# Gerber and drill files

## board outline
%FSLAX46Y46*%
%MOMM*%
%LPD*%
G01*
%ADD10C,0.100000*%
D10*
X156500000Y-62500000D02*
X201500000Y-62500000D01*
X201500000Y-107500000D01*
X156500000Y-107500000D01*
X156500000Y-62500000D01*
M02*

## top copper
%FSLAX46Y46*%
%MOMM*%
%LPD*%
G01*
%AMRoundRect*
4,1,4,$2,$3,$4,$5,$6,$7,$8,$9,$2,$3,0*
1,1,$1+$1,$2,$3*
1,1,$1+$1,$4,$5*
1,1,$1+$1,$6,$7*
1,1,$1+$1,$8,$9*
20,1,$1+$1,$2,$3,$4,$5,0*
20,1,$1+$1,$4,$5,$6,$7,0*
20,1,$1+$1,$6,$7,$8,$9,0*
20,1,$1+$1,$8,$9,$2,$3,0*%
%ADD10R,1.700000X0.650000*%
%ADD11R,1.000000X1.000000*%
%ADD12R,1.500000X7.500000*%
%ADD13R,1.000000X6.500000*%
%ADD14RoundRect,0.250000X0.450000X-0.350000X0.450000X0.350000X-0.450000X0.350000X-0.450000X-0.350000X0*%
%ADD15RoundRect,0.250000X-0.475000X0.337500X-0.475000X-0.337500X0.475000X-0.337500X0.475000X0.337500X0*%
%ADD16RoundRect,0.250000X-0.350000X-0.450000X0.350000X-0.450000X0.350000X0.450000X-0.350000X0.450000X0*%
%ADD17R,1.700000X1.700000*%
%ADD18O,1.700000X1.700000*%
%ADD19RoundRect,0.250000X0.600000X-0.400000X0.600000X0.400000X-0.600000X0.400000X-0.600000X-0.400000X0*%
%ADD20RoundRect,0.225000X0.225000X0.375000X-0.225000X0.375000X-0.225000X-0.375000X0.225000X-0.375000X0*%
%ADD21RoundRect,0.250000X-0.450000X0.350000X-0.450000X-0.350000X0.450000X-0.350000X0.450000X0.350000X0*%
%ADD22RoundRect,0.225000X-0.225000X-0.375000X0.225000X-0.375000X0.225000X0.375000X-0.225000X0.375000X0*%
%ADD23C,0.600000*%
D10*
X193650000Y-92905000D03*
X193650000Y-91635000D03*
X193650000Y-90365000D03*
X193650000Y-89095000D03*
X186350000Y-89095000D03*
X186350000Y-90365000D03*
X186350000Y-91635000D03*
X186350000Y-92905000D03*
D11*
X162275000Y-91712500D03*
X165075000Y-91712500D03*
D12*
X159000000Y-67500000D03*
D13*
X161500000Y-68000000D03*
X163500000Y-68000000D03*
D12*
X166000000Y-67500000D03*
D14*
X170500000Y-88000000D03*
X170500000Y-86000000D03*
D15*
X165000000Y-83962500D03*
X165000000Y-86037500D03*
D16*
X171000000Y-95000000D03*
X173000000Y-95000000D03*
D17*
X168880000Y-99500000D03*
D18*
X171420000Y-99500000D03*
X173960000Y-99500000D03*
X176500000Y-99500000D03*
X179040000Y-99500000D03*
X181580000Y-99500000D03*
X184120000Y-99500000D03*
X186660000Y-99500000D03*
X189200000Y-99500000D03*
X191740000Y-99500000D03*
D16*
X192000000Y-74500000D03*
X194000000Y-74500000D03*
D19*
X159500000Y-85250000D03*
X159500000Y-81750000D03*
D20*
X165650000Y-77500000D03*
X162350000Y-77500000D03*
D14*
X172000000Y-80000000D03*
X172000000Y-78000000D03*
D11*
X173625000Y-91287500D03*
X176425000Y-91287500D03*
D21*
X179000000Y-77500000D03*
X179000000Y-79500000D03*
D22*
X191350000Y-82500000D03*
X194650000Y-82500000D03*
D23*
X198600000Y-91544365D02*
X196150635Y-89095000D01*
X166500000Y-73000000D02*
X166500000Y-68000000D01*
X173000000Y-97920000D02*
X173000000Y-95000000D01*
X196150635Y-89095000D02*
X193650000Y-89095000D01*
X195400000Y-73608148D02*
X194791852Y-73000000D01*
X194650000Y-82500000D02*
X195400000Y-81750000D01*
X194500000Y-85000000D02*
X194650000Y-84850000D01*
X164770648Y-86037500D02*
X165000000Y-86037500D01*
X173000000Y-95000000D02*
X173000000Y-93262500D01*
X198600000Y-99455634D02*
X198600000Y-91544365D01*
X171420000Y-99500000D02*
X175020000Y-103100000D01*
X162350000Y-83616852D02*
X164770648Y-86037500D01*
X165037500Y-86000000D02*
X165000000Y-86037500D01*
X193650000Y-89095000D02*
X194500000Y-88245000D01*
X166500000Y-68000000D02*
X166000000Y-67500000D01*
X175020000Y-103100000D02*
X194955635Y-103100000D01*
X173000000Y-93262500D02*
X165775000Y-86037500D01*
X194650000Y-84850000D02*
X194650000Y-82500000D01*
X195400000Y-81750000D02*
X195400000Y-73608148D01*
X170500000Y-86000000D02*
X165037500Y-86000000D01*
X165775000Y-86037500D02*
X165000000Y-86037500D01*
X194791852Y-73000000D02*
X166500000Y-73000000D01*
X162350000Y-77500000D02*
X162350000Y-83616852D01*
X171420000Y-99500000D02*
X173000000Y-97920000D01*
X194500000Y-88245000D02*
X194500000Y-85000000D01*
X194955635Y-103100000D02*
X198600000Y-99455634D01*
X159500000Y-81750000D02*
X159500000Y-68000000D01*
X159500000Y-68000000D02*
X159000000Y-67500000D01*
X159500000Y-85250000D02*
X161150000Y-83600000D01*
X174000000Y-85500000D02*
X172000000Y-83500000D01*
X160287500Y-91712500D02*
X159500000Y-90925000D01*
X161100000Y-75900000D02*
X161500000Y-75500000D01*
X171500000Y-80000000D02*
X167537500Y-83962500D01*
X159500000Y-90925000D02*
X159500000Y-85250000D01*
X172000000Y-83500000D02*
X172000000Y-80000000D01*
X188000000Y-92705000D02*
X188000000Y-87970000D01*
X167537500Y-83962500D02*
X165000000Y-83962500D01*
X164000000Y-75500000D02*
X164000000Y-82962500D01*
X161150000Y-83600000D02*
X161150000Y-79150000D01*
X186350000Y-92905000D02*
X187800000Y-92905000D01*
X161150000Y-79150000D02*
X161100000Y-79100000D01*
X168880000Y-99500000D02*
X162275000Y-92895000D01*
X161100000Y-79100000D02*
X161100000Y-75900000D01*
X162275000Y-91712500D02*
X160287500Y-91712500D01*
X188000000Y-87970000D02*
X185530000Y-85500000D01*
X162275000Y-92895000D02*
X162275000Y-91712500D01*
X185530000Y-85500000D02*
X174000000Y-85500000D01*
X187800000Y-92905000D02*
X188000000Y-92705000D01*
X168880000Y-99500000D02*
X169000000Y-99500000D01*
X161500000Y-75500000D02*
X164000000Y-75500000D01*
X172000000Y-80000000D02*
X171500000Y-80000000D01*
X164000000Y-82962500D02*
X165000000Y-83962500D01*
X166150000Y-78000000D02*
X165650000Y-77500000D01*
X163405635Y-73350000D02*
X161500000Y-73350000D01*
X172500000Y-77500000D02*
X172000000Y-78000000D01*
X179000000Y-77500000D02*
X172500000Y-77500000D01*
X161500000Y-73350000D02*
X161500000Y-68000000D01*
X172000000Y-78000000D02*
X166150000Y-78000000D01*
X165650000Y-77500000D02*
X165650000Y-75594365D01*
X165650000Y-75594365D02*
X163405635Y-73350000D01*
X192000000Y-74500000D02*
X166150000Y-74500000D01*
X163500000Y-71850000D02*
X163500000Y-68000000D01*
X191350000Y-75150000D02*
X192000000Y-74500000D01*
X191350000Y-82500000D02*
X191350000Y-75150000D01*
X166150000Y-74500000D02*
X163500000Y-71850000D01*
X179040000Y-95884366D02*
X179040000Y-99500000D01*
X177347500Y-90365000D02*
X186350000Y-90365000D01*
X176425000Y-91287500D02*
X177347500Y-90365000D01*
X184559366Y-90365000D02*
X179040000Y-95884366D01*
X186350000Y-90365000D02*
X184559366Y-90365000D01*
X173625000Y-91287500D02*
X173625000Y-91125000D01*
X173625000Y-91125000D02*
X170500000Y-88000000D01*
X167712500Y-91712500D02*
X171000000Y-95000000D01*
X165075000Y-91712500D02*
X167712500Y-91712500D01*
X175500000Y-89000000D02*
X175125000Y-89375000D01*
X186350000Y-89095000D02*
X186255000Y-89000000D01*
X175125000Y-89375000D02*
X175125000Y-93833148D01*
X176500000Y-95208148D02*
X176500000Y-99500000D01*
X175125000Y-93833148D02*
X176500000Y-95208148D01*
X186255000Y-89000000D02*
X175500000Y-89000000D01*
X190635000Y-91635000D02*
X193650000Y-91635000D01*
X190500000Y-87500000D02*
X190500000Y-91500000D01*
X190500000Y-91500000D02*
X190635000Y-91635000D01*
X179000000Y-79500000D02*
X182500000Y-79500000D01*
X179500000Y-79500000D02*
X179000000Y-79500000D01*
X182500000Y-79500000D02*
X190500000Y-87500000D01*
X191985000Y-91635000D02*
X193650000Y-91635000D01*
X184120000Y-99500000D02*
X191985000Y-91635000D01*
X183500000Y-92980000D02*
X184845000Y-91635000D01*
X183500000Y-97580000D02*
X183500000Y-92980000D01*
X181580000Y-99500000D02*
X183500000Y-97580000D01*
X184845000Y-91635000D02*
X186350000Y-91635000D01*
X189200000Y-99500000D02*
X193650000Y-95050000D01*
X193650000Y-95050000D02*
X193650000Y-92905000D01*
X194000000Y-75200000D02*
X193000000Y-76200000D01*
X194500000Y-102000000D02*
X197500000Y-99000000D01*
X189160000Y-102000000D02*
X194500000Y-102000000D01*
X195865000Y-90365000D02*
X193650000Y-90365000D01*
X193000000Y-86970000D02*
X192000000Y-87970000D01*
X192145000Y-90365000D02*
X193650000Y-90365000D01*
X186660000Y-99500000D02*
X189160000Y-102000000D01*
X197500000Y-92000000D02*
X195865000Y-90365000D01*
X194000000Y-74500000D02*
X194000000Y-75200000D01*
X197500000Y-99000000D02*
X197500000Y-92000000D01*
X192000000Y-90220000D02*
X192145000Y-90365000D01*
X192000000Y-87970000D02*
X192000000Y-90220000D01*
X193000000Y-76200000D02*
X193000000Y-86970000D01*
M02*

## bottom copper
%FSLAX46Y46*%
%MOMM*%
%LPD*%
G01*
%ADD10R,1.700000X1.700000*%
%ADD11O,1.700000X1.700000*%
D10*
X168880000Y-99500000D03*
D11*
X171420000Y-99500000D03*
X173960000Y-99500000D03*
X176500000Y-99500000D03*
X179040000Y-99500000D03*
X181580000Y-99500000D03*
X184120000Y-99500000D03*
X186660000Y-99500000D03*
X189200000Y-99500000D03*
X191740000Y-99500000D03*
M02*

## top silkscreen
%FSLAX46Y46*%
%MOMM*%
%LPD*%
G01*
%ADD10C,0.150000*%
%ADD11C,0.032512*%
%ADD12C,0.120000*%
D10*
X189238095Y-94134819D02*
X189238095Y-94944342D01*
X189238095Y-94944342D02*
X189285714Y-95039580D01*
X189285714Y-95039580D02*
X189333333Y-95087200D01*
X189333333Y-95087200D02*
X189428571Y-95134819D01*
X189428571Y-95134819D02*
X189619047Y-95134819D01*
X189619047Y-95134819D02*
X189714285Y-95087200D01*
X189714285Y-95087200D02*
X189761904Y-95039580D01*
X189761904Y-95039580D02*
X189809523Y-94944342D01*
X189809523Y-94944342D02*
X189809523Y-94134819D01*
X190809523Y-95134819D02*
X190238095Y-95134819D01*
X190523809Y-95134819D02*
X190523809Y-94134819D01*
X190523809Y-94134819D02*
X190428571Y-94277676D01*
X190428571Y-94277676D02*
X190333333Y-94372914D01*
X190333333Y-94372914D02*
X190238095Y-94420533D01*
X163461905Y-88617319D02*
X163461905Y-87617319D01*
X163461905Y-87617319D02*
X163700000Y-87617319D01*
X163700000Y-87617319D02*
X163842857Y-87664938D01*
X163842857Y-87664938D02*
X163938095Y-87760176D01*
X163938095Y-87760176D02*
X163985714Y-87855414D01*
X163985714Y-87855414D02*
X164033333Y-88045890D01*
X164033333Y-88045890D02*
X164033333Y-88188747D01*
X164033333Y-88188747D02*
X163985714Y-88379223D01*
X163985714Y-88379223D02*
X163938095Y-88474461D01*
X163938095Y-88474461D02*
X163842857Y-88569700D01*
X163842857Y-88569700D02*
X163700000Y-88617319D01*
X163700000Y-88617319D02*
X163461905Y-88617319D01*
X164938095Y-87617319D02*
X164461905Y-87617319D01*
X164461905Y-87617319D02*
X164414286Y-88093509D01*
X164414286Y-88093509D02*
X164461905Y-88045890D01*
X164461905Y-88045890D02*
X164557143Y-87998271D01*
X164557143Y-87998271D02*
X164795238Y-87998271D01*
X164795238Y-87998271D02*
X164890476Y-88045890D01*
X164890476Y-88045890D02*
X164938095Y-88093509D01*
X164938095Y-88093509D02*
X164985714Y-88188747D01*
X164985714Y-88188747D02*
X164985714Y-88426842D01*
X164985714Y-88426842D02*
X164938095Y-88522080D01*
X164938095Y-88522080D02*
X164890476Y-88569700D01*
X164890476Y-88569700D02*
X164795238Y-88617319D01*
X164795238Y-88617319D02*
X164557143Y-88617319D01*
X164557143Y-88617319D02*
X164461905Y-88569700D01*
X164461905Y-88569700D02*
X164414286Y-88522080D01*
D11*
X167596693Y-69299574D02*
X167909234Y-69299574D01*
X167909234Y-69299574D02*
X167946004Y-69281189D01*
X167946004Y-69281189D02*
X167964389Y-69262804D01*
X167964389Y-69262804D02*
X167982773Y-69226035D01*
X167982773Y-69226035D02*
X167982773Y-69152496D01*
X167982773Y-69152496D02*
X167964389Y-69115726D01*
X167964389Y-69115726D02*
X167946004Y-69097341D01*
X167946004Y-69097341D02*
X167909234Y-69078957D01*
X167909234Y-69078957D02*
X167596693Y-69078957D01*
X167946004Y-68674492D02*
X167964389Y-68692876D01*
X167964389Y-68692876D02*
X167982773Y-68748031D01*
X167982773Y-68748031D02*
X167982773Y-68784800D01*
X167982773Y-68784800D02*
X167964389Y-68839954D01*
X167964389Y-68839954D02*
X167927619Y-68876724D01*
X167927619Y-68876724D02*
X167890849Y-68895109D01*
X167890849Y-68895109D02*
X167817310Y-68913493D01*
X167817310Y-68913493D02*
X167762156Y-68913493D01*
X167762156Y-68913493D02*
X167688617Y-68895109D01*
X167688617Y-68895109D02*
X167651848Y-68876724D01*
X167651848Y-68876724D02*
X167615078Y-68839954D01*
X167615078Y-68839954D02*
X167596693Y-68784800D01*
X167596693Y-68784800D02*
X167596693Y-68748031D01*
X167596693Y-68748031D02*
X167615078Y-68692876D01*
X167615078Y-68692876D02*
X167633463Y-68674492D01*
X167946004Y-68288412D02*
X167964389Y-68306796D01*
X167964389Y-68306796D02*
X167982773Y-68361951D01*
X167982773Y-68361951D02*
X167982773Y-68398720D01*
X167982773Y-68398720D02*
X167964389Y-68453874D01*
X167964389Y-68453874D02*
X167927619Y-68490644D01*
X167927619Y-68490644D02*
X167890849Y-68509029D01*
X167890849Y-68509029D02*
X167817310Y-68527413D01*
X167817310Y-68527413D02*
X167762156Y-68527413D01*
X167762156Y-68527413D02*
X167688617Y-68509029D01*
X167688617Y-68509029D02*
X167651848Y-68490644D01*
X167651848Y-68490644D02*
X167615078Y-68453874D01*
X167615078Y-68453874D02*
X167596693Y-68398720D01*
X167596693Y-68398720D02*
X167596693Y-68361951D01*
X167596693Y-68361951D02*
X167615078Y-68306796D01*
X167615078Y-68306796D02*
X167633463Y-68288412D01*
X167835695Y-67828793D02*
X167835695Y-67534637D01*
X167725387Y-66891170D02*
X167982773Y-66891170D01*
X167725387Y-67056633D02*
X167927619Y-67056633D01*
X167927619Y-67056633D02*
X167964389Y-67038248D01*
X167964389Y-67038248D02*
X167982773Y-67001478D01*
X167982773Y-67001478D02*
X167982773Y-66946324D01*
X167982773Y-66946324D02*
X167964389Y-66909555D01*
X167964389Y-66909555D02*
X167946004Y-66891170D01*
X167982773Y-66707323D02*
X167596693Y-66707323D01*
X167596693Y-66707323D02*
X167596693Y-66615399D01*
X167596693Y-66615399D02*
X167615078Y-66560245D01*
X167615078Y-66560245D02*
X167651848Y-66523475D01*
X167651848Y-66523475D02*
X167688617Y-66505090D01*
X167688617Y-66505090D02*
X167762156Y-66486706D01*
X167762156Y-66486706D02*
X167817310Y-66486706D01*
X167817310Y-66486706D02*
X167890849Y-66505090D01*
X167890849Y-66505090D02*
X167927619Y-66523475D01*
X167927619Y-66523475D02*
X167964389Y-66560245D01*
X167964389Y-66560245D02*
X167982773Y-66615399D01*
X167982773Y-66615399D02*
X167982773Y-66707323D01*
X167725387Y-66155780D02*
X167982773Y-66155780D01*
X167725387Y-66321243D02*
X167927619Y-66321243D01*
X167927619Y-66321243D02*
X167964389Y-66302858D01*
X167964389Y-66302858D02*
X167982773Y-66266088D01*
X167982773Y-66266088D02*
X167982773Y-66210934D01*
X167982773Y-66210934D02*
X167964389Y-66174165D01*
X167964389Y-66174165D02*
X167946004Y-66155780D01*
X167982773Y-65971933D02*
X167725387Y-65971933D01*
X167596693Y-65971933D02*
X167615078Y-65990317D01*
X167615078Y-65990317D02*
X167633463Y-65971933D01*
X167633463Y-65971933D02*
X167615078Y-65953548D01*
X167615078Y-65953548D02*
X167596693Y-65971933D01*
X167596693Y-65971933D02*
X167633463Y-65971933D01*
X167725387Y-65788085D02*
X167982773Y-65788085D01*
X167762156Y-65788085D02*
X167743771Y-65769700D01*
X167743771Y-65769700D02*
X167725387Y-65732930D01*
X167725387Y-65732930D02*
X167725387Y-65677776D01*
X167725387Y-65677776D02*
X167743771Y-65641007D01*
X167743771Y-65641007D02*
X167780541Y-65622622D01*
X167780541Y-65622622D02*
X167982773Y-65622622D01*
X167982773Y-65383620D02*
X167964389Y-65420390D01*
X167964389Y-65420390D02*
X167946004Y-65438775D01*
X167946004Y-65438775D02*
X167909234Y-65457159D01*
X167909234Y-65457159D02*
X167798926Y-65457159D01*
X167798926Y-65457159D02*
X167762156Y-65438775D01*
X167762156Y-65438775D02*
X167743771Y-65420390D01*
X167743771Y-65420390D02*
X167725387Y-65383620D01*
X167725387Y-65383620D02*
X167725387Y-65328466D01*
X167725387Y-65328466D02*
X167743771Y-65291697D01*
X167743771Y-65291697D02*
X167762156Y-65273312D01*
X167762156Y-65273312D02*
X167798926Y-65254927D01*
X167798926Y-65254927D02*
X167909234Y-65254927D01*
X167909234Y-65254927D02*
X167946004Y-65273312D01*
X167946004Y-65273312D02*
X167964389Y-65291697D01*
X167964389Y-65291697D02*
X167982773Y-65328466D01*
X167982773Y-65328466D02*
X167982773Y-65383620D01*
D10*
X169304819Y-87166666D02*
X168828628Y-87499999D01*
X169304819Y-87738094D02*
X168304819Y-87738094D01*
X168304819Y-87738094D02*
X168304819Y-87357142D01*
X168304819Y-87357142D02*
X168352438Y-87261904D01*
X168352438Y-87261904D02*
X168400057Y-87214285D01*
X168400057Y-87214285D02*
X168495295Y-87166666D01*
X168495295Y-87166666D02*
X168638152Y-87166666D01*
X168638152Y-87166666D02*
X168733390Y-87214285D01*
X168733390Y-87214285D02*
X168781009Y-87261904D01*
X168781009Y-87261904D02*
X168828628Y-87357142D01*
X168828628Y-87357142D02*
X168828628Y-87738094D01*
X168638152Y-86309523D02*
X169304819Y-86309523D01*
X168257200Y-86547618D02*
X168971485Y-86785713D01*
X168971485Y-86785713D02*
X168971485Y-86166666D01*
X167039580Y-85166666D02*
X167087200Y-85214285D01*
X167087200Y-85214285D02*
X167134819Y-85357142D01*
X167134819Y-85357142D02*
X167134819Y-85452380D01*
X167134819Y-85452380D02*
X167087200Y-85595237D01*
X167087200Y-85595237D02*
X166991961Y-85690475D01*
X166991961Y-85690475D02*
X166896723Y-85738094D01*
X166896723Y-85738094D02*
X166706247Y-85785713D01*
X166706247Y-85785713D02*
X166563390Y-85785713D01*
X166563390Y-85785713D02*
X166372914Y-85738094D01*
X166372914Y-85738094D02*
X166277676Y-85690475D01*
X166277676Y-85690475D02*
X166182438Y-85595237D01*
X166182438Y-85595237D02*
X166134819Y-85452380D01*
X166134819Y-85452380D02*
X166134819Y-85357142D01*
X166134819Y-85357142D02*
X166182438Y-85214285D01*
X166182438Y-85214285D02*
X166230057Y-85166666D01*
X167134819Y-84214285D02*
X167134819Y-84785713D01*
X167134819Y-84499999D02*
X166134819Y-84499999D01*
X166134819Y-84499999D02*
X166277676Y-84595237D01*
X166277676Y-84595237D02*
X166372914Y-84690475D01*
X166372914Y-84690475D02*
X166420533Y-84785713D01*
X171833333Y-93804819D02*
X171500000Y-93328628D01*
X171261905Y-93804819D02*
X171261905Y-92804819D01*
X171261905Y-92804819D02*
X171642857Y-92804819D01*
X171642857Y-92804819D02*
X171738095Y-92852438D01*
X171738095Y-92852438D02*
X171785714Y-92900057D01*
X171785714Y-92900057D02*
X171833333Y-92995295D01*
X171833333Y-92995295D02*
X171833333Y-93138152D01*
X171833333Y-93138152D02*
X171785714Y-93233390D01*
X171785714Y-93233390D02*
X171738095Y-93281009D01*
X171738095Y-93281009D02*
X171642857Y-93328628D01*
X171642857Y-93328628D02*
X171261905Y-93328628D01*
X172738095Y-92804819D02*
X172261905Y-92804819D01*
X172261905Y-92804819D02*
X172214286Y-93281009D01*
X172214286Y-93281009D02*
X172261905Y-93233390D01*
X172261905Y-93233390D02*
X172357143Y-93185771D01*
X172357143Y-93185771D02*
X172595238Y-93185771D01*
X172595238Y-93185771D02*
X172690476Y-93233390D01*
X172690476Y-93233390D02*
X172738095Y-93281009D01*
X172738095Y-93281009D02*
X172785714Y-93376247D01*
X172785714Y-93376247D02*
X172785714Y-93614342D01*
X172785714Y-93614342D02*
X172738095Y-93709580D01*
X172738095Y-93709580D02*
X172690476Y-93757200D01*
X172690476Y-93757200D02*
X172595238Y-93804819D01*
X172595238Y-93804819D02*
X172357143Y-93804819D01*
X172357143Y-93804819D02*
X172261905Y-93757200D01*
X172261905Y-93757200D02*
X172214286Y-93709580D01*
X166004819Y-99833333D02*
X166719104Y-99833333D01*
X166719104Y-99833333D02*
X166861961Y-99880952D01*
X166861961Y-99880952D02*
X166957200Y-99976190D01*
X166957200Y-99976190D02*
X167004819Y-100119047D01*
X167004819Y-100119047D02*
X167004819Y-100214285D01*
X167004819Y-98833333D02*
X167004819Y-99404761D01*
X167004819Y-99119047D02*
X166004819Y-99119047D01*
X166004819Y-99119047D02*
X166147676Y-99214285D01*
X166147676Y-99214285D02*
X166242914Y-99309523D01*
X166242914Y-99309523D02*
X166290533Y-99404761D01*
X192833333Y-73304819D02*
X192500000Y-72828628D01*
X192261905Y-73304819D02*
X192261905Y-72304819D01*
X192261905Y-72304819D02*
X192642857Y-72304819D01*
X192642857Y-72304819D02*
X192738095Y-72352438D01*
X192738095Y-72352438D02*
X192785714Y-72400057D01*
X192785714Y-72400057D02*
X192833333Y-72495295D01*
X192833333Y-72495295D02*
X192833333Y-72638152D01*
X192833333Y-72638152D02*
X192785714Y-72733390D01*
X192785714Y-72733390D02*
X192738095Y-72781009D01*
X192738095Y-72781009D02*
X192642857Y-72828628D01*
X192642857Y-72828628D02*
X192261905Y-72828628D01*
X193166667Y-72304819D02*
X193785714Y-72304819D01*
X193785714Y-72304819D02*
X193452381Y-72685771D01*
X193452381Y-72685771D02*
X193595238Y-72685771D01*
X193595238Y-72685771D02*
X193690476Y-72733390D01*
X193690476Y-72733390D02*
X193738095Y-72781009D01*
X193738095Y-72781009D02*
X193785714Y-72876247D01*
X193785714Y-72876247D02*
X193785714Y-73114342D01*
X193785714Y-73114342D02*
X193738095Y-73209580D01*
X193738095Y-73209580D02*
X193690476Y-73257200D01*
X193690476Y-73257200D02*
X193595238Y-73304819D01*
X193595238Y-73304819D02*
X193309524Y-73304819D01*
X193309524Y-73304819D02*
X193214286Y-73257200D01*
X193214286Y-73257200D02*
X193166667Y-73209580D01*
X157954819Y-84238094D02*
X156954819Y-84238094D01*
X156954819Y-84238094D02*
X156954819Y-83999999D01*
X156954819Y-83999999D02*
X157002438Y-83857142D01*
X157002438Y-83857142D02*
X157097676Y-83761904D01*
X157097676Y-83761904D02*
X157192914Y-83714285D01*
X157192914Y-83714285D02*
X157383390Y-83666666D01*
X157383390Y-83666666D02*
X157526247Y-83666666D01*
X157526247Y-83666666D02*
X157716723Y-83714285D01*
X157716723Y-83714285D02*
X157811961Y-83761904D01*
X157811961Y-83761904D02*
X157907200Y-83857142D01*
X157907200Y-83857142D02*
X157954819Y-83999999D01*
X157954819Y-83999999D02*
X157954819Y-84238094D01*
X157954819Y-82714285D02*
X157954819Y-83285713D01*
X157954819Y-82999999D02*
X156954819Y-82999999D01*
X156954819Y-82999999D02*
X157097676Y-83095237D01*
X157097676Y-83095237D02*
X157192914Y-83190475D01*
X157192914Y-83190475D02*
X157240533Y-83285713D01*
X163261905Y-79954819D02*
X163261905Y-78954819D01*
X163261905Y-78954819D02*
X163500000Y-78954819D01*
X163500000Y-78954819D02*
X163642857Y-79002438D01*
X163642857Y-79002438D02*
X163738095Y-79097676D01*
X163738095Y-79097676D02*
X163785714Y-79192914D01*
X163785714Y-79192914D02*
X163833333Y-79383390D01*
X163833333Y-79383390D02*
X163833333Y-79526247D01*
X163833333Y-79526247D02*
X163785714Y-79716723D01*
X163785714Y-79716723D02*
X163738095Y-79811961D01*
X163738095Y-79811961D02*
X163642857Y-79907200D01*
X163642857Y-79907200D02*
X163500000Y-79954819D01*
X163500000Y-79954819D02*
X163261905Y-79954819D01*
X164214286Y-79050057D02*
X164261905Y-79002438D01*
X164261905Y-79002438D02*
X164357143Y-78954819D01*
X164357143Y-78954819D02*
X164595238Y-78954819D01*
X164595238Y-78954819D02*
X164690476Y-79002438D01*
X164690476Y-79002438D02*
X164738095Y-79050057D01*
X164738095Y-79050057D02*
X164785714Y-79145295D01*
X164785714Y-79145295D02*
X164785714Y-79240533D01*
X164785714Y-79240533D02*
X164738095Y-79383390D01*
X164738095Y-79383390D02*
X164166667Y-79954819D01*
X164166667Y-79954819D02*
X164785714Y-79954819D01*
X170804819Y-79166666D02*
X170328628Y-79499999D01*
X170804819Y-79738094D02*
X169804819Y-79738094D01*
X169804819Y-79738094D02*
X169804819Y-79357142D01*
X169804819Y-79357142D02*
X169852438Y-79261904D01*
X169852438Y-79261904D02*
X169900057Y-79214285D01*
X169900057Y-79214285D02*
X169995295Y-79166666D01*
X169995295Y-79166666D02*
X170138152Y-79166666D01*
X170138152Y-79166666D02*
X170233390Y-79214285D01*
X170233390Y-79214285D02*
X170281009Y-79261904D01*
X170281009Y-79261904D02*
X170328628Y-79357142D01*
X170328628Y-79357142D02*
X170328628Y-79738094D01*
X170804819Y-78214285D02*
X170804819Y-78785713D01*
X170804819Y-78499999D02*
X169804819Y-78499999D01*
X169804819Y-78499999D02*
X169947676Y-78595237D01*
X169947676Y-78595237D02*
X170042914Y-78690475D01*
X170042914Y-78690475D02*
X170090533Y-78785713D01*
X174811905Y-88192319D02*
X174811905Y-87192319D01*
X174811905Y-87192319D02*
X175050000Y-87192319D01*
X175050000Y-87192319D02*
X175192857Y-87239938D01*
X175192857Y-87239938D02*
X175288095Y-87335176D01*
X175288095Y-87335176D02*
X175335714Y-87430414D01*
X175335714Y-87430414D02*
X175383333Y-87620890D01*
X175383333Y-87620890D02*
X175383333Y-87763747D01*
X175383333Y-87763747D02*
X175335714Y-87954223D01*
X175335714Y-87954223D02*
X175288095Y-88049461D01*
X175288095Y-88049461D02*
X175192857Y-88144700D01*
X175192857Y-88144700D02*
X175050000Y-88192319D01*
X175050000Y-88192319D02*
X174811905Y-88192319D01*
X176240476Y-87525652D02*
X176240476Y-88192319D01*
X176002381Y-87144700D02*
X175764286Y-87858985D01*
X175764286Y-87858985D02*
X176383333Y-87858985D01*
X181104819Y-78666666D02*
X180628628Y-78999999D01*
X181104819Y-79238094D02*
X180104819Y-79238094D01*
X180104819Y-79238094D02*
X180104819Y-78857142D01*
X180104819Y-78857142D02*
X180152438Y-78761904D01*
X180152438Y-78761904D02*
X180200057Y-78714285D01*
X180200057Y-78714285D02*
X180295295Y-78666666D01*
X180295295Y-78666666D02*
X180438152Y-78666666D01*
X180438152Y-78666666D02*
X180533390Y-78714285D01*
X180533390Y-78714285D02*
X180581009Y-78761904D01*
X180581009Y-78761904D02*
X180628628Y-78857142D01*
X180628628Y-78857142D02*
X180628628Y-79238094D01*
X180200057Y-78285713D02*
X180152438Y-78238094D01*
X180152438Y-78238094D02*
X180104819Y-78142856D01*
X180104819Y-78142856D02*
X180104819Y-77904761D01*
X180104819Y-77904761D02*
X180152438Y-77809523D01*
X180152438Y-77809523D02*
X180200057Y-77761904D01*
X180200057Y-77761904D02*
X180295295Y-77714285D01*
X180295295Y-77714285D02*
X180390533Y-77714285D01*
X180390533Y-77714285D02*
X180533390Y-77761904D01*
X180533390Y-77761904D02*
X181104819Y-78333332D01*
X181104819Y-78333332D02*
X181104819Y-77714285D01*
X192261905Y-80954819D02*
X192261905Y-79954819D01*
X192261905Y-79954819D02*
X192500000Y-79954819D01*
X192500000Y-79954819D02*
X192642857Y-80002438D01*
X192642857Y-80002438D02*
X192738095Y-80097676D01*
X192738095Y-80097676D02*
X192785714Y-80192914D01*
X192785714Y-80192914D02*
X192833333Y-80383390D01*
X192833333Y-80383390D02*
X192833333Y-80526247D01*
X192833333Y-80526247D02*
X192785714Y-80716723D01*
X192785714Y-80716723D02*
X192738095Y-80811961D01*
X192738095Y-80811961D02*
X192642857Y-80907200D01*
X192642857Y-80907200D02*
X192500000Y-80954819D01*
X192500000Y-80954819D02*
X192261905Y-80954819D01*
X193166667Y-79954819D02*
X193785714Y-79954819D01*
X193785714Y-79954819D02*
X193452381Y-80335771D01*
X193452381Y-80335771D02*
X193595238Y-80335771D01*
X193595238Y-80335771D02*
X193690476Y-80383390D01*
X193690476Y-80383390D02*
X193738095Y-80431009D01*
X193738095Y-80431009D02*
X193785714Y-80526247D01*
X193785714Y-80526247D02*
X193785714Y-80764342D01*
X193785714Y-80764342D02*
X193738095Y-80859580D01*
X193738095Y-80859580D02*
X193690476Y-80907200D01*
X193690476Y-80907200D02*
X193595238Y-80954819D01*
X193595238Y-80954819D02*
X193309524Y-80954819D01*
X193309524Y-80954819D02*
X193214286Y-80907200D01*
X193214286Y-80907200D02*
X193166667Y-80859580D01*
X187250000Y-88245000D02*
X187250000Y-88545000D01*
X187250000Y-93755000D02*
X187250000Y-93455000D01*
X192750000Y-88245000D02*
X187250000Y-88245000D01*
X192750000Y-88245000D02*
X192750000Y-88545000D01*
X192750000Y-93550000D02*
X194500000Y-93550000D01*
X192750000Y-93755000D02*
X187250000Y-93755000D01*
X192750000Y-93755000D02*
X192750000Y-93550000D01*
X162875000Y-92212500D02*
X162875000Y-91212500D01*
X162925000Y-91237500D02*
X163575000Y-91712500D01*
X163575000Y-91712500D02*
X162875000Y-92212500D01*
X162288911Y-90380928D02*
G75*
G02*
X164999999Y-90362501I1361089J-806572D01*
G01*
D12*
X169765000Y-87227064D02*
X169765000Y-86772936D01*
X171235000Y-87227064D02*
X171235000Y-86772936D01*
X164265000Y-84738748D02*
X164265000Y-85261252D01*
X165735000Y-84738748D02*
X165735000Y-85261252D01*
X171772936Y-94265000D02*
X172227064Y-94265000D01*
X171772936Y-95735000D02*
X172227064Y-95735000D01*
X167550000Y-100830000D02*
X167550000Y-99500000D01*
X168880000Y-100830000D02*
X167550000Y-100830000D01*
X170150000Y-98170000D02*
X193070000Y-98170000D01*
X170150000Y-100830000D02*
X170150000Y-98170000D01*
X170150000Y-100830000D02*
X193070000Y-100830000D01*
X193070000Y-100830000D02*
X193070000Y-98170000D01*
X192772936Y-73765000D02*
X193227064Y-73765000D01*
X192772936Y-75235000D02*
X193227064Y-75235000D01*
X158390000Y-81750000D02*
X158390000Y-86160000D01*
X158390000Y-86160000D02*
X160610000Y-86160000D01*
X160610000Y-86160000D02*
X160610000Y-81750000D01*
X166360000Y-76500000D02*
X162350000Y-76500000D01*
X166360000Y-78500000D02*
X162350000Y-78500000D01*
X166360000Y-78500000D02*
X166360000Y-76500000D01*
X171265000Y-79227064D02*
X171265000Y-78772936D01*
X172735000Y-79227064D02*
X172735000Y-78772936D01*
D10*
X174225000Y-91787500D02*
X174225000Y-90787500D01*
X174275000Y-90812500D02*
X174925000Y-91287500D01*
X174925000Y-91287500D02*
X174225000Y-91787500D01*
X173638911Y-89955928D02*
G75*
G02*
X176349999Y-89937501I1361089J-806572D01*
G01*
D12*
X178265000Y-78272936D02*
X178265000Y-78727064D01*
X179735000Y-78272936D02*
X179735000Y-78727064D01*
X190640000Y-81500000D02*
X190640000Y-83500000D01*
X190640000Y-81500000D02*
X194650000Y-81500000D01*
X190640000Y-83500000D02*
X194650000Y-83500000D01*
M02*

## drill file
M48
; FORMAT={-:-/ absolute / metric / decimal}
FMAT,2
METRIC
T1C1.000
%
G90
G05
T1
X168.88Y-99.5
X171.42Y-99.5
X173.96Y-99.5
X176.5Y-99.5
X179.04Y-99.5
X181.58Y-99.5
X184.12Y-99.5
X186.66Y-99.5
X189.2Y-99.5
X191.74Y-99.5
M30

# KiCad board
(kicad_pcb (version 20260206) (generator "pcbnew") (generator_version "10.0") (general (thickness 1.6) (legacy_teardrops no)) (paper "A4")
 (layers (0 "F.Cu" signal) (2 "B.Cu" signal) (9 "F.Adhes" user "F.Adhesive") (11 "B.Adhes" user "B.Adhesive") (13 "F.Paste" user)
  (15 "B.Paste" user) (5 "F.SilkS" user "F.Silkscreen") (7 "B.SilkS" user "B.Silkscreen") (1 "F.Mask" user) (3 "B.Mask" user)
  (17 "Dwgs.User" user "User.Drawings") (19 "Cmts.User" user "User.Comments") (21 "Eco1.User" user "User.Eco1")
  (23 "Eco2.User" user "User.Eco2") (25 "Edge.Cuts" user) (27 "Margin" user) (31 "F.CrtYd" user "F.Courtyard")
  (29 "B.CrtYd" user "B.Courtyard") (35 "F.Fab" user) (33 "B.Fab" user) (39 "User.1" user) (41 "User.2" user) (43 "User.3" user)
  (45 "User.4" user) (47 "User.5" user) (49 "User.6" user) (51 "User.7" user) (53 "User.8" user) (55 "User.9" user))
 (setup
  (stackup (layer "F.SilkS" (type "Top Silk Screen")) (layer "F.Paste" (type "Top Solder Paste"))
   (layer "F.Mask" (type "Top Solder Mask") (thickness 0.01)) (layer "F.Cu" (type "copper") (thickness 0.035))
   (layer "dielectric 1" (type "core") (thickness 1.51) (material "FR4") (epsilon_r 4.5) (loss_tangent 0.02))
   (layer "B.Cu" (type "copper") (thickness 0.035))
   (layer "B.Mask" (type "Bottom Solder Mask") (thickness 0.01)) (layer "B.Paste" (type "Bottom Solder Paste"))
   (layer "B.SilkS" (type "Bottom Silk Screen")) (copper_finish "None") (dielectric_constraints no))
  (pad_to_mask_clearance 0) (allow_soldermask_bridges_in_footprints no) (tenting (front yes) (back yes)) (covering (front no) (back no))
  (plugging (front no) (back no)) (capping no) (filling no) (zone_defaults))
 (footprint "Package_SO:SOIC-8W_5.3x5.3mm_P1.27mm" (layer "F.Cu") (at 190 91 180)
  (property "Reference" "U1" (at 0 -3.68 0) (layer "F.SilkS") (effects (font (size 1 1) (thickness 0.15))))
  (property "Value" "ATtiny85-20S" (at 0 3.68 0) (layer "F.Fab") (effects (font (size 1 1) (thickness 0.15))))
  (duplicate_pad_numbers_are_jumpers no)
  (fp_line (start 2.75 2.755) (end 2.75 2.455) (stroke (width 0.15) (type solid)) (layer "F.SilkS"))
  (fp_line (start 2.75 -2.755) (end 2.75 -2.455) (stroke (width 0.15) (type solid)) (layer "F.SilkS"))
  (fp_line (start -2.75 2.755) (end 2.75 2.755) (stroke (width 0.15) (type solid)) (layer "F.SilkS"))
  (fp_line (start -2.75 2.755) (end -2.75 2.455) (stroke (width 0.15) (type solid)) (layer "F.SilkS"))
  (fp_line (start -2.75 -2.55) (end -4.5 -2.55) (stroke (width 0.15) (type solid)) (layer "F.SilkS"))
  (fp_line (start -2.75 -2.755) (end 2.75 -2.755) (stroke (width 0.15) (type solid)) (layer "F.SilkS"))
  (fp_line (start -2.75 -2.755) (end -2.75 -2.55) (stroke (width 0.15) (type solid)) (layer "F.SilkS"))
  (pad "1" smd rect (at -3.65 -1.905 180) (size 1.7 0.65) (layers "F.Cu" "F.Mask" "F.Paste") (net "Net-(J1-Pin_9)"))
  (pad "2" smd rect (at -3.65 -0.635 180) (size 1.7 0.65) (layers "F.Cu" "F.Mask" "F.Paste") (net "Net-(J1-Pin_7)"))
  (pad "3" smd rect (at -3.65 0.635 180) (size 1.7 0.65) (layers "F.Cu" "F.Mask" "F.Paste") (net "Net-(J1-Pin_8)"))
  (pad "4" smd rect (at -3.65 1.905 180) (size 1.7 0.65) (layers "F.Cu" "F.Mask" "F.Paste") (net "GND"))
  (pad "5" smd rect (at 3.65 1.905 180) (size 1.7 0.65) (layers "F.Cu" "F.Mask" "F.Paste") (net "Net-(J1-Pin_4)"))
  (pad "6" smd rect (at 3.65 0.635 180) (size 1.7 0.65) (layers "F.Cu" "F.Mask" "F.Paste") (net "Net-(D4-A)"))
  (pad "7" smd rect (at 3.65 -0.635 180) (size 1.7 0.65) (layers "F.Cu" "F.Mask" "F.Paste") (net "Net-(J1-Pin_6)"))
  (pad "8" smd rect (at 3.65 -1.905 180) (size 1.7 0.65) (layers "F.Cu" "F.Mask" "F.Paste") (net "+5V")))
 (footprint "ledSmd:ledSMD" (layer "F.Cu") (at 164.075 91.7125)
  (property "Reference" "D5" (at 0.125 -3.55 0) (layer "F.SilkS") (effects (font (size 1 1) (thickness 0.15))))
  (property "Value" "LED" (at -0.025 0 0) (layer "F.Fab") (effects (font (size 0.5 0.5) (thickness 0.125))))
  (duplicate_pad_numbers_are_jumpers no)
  (fp_line (start -1.2 0.5) (end -1.2 -0.5) (stroke (width 0.15) (type solid)) (layer "F.SilkS"))
  (fp_line (start -1.15 -0.475) (end -0.5 0) (stroke (width 0.15) (type solid)) (layer "F.SilkS"))
  (fp_line (start -0.5 0) (end -1.2 0.5) (stroke (width 0.15) (type solid)) (layer "F.SilkS"))
  (fp_arc (start -1.786089 -1.331572) (mid -0.435753 -2.107089) (end 0.924999 -1.349999) (stroke (width 0.15) (type solid))
   (layer "F.SilkS"))
  (pad "1" smd rect (at -1.8 0) (size 1 1) (layers "F.Cu" "F.Mask" "F.Paste") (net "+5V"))
  (pad "2" smd rect (at 1 0) (size 1 1) (layers "F.Cu" "F.Mask" "F.Paste") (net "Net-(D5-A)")))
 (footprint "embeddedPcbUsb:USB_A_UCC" (layer "F.Cu") (at 162.5 67.7 -90)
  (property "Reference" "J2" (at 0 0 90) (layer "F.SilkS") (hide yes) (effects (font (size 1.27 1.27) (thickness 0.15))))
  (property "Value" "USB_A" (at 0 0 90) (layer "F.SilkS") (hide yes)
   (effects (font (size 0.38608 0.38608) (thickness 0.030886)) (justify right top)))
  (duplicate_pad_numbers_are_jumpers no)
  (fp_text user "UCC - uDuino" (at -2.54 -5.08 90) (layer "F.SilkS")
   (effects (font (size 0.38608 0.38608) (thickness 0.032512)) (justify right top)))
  (pad "1" smd rect (at -0.2 3.5 270) (size 7.5 1.5) (layers "F.Cu" "F.Mask" "F.Paste") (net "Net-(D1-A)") (solder_mask_margin 0.1016))
  (pad "2" smd rect (at 0.3 1 270) (size 6.5 1) (layers "F.Cu" "F.Mask" "F.Paste") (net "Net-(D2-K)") (solder_mask_margin 0.1016))
  (pad "3" smd rect (at 0.3 -1 270) (size 6.5 1) (layers "F.Cu" "F.Mask" "F.Paste") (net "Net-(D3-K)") (solder_mask_margin 0.1016))
  (pad "4" smd rect (at -0.2 -3.5 270) (size 7.5 1.5) (layers "F.Cu" "F.Mask" "F.Paste") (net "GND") (solder_mask_margin 0.1016)))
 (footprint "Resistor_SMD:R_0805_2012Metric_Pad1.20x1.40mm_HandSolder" (layer "F.Cu") (at 170.5 87 90)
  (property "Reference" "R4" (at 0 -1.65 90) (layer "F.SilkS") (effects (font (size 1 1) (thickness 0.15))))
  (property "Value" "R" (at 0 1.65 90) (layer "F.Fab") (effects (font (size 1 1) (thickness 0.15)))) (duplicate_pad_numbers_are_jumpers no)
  (fp_line (start -0.227064 -0.735) (end 0.227064 -0.735) (stroke (width 0.12) (type solid)) (layer "F.SilkS"))
  (fp_line (start -0.227064 0.735) (end 0.227064 0.735) (stroke (width 0.12) (type solid)) (layer "F.SilkS"))
  (pad "1" smd roundrect (at -1 0 90) (size 1.2 1.4) (layers "F.Cu" "F.Mask" "F.Paste") (roundrect_rratio 0.208333) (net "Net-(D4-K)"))
  (pad "2" smd roundrect (at 1 0 90) (size 1.2 1.4) (layers "F.Cu" "F.Mask" "F.Paste") (roundrect_rratio 0.208333) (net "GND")))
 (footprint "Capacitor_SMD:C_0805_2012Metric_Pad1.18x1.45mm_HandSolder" (layer "F.Cu") (at 165 85 -90)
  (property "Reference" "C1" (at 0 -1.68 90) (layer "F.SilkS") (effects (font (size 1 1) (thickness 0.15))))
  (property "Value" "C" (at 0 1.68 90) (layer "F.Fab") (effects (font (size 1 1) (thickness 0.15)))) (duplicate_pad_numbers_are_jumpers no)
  (fp_line (start -0.261252 0.735) (end 0.261252 0.735) (stroke (width 0.12) (type solid)) (layer "F.SilkS"))
  (fp_line (start -0.261252 -0.735) (end 0.261252 -0.735) (stroke (width 0.12) (type solid)) (layer "F.SilkS"))
  (pad "1" smd roundrect (at -1.0375 0 270) (size 1.175 1.45) (layers "F.Cu" "F.Mask" "F.Paste") (roundrect_rratio 0.212766) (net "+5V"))
  (pad "2" smd roundrect (at 1.0375 0 270) (size 1.175 1.45) (layers "F.Cu" "F.Mask" "F.Paste") (roundrect_rratio 0.212766) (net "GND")))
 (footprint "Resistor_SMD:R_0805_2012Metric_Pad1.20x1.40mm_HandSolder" (layer "F.Cu") (at 172 95)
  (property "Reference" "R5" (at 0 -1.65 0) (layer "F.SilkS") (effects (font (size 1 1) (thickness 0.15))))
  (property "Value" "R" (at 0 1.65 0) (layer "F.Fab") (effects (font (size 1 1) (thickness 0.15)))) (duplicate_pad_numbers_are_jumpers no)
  (fp_line (start -0.227064 -0.735) (end 0.227064 -0.735) (stroke (width 0.12) (type solid)) (layer "F.SilkS"))
  (fp_line (start -0.227064 0.735) (end 0.227064 0.735) (stroke (width 0.12) (type solid)) (layer "F.SilkS"))
  (pad "1" smd roundrect (at -1 0) (size 1.2 1.4) (layers "F.Cu" "F.Mask" "F.Paste") (roundrect_rratio 0.208333) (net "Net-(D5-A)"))
  (pad "2" smd roundrect (at 1 0) (size 1.2 1.4) (layers "F.Cu" "F.Mask" "F.Paste") (roundrect_rratio 0.208333) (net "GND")))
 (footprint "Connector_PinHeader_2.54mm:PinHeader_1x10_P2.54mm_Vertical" (layer "F.Cu") (at 168.88 99.5 90)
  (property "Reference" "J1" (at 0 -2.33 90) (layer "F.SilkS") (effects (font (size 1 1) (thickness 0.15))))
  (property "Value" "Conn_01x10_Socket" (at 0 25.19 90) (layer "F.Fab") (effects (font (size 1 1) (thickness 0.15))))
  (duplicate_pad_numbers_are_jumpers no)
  (fp_line (start -1.33 -1.33) (end 0 -1.33) (stroke (width 0.12) (type solid)) (layer "F.SilkS"))
  (fp_line (start -1.33 0) (end -1.33 -1.33) (stroke (width 0.12) (type solid)) (layer "F.SilkS"))
  (fp_line (start 1.33 1.27) (end 1.33 24.19) (stroke (width 0.12) (type solid)) (layer "F.SilkS"))
  (fp_line (start -1.33 1.27) (end 1.33 1.27) (stroke (width 0.12) (type solid)) (layer "F.SilkS"))
  (fp_line (start -1.33 1.27) (end -1.33 24.19) (stroke (width 0.12) (type solid)) (layer "F.SilkS"))
  (fp_line (start -1.33 24.19) (end 1.33 24.19) (stroke (width 0.12) (type solid)) (layer "F.SilkS"))
  (pad "1" thru_hole rect (at 0 0 90) (size 1.7 1.7) (drill 1) (layers "*.Cu" "*.Mask") (remove_unused_layers no) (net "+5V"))
  (pad "2" thru_hole oval (at 0 2.54 90) (size 1.7 1.7) (drill 1) (layers "*.Cu" "*.Mask") (remove_unused_layers no) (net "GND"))
  (pad "3" thru_hole oval (at 0 5.08 90) (size 1.7 1.7) (drill 1) (layers "*.Cu" "*.Mask") (remove_unused_layers no)
   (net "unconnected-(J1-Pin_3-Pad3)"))
  (pad "4" thru_hole oval (at 0 7.62 90) (size 1.7 1.7) (drill 1) (layers "*.Cu" "*.Mask") (remove_unused_layers no) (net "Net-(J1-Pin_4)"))
  (pad "5" thru_hole oval (at 0 10.16 90) (size 1.7 1.7) (drill 1) (layers "*.Cu" "*.Mask") (remove_unused_layers no) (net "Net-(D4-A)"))
  (pad "6" thru_hole oval (at 0 12.7 90) (size 1.7 1.7) (drill 1) (layers "*.Cu" "*.Mask") (remove_unused_layers no) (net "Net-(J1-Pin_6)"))
  (pad "7" thru_hole oval (at 0 15.24 90) (size 1.7 1.7) (drill 1) (layers "*.Cu" "*.Mask") (remove_unused_layers no) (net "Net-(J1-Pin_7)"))
  (pad "8" thru_hole oval (at 0 17.78 90) (size 1.7 1.7) (drill 1) (layers "*.Cu" "*.Mask") (remove_unused_layers no) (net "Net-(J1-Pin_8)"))
  (pad "9" thru_hole oval (at 0 20.32 90) (size 1.7 1.7) (drill 1) (layers "*.Cu" "*.Mask") (remove_unused_layers no) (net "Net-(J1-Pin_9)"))
  (pad "10" thru_hole oval (at 0 22.86 90) (size 1.7 1.7) (drill 1) (layers "*.Cu" "*.Mask") (remove_unused_layers no)
   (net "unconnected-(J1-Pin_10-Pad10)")))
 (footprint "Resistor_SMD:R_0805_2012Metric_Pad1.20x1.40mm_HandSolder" (layer "F.Cu") (at 193 74.5)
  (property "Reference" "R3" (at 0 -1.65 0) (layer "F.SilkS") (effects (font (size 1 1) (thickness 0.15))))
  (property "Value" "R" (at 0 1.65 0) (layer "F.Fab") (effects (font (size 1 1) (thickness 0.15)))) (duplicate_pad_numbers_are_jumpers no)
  (fp_line (start -0.227064 -0.735) (end 0.227064 -0.735) (stroke (width 0.12) (type solid)) (layer "F.SilkS"))
  (fp_line (start -0.227064 0.735) (end 0.227064 0.735) (stroke (width 0.12) (type solid)) (layer "F.SilkS"))
  (pad "1" smd roundrect (at -1 0) (size 1.2 1.4) (layers "F.Cu" "F.Mask" "F.Paste") (roundrect_rratio 0.208333) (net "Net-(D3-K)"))
  (pad "2" smd roundrect (at 1 0) (size 1.2 1.4) (layers "F.Cu" "F.Mask" "F.Paste") (roundrect_rratio 0.208333) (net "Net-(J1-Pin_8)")))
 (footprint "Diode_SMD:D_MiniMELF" (layer "F.Cu") (at 159.5 83.5 90)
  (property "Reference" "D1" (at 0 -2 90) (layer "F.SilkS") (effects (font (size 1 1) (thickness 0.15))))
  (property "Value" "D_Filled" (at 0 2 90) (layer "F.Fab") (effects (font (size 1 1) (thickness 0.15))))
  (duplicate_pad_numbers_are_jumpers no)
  (fp_line (start 1.75 -1.11) (end -2.66 -1.11) (stroke (width 0.12) (type solid)) (layer "F.SilkS"))
  (fp_line (start -2.66 -1.11) (end -2.66 1.11) (stroke (width 0.12) (type solid)) (layer "F.SilkS"))
  (fp_line (start -2.66 1.11) (end 1.75 1.11) (stroke (width 0.12) (type solid)) (layer "F.SilkS"))
  (pad "1" smd roundrect (at -1.75 0 90) (size 1.3 1.7) (layers "F.Cu" "F.Mask" "F.Paste") (roundrect_rratio 0.1923076923) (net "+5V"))
  (pad "2" smd roundrect (at 1.75 0 90) (size 1.3 1.7) (layers "F.Cu" "F.Mask" "F.Paste") (roundrect_rratio 0.1923076923) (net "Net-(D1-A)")))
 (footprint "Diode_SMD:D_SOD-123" (layer "F.Cu") (at 164 77.5 180)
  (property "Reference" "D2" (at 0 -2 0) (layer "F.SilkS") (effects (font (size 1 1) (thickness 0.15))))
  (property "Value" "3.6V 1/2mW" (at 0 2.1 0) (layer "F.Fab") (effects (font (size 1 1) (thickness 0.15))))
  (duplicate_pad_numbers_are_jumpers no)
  (fp_line (start -2.36 1) (end 1.65 1) (stroke (width 0.12) (type solid)) (layer "F.SilkS"))
  (fp_line (start -2.36 -1) (end 1.65 -1) (stroke (width 0.12) (type solid)) (layer "F.SilkS"))
  (fp_line (start -2.36 -1) (end -2.36 1) (stroke (width 0.12) (type solid)) (layer "F.SilkS"))
  (pad "1" smd roundrect (at -1.65 0 180) (size 0.9 1.2) (layers "F.Cu" "F.Mask" "F.Paste") (roundrect_rratio 0.25) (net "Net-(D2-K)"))
  (pad "2" smd roundrect (at 1.65 0 180) (size 0.9 1.2) (layers "F.Cu" "F.Mask" "F.Paste") (roundrect_rratio 0.25) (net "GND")))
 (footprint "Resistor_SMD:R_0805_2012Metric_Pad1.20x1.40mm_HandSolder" (layer "F.Cu") (at 172 79 90)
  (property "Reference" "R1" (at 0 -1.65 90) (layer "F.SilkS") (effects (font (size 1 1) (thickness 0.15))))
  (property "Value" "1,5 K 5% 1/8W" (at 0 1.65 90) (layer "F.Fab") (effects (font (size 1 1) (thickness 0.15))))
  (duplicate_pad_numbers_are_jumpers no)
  (fp_line (start -0.227064 -0.735) (end 0.227064 -0.735) (stroke (width 0.12) (type solid)) (layer "F.SilkS"))
  (fp_line (start -0.227064 0.735) (end 0.227064 0.735) (stroke (width 0.12) (type solid)) (layer "F.SilkS"))
  (pad "1" smd roundrect (at -1 0 90) (size 1.2 1.4) (layers "F.Cu" "F.Mask" "F.Paste") (roundrect_rratio 0.208333) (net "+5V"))
  (pad "2" smd roundrect (at 1 0 90) (size 1.2 1.4) (layers "F.Cu" "F.Mask" "F.Paste") (roundrect_rratio 0.208333) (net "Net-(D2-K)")))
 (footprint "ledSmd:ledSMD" (layer "F.Cu") (at 175.425 91.2875)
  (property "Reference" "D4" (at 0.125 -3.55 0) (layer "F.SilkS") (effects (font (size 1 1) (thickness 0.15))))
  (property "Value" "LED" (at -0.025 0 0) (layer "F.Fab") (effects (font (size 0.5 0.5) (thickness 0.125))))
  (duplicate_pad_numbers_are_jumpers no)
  (fp_line (start -1.2 0.5) (end -1.2 -0.5) (stroke (width 0.15) (type solid)) (layer "F.SilkS"))
  (fp_line (start -1.15 -0.475) (end -0.5 0) (stroke (width 0.15) (type solid)) (layer "F.SilkS"))
  (fp_line (start -0.5 0) (end -1.2 0.5) (stroke (width 0.15) (type solid)) (layer "F.SilkS"))
  (fp_arc (start -1.786089 -1.331572) (mid -0.435753 -2.107089) (end 0.924999 -1.349999) (stroke (width 0.15) (type solid))
   (layer "F.SilkS"))
  (pad "1" smd rect (at -1.8 0) (size 1 1) (layers "F.Cu" "F.Mask" "F.Paste") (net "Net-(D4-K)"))
  (pad "2" smd rect (at 1 0) (size 1 1) (layers "F.Cu" "F.Mask" "F.Paste") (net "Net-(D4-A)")))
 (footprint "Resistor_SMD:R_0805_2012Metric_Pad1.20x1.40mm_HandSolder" (layer "F.Cu") (at 179 78.5 -90)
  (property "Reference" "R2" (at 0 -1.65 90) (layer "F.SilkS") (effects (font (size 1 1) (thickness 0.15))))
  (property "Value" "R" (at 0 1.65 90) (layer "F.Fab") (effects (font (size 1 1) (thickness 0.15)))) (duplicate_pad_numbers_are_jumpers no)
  (fp_line (start -0.227064 0.735) (end 0.227064 0.735) (stroke (width 0.12) (type solid)) (layer "F.SilkS"))
  (fp_line (start -0.227064 -0.735) (end 0.227064 -0.735) (stroke (width 0.12) (type solid)) (layer "F.SilkS"))
  (pad "1" smd roundrect (at -1 0 270) (size 1.2 1.4) (layers "F.Cu" "F.Mask" "F.Paste") (roundrect_rratio 0.208333) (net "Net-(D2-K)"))
  (pad "2" smd roundrect (at 1 0 270) (size 1.2 1.4) (layers "F.Cu" "F.Mask" "F.Paste") (roundrect_rratio 0.208333) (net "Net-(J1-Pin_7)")))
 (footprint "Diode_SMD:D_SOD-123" (layer "F.Cu") (at 193 82.5)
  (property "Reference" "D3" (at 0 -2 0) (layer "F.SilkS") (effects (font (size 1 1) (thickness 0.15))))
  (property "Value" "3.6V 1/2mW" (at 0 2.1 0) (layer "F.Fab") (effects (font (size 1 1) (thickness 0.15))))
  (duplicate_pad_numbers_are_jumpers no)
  (fp_line (start -2.36 -1) (end -2.36 1) (stroke (width 0.12) (type solid)) (layer "F.SilkS"))
  (fp_line (start -2.36 -1) (end 1.65 -1) (stroke (width 0.12) (type solid)) (layer "F.SilkS"))
  (fp_line (start -2.36 1) (end 1.65 1) (stroke (width 0.12) (type solid)) (layer "F.SilkS"))
  (pad "1" smd roundrect (at -1.65 0) (size 0.9 1.2) (layers "F.Cu" "F.Mask" "F.Paste") (roundrect_rratio 0.25) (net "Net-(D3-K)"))
  (pad "2" smd roundrect (at 1.65 0) (size 0.9 1.2) (layers "F.Cu" "F.Mask" "F.Paste") (roundrect_rratio 0.25) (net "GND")))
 (gr_rect (start 156.5 62.5) (end 201.5 107.5) (stroke (width 0.1) (type default)) (fill no) (layer "Edge.Cuts"))
 (segment (start 198.6 91.544365) (end 196.150635 89.095) (width 0.6) (layer "F.Cu") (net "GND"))
 (segment (start 166.5 73) (end 166.5 68) (width 0.6) (layer "F.Cu") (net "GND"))
 (segment (start 173 97.92) (end 173 95) (width 0.6) (layer "F.Cu") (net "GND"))
 (segment (start 196.150635 89.095) (end 193.65 89.095) (width 0.6) (layer "F.Cu") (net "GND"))
 (segment (start 195.4 73.608148) (end 194.791852 73) (width 0.6) (layer "F.Cu") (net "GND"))
 (segment (start 194.65 82.5) (end 195.4 81.75) (width 0.6) (layer "F.Cu") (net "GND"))
 (segment (start 194.5 85) (end 194.65 84.85) (width 0.6) (layer "F.Cu") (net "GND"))
 (segment (start 164.770648 86.0375) (end 165 86.0375) (width 0.6) (layer "F.Cu") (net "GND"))
 (segment (start 173 95) (end 173 93.2625) (width 0.6) (layer "F.Cu") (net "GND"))
 (segment (start 198.6 99.455634) (end 198.6 91.544365) (width 0.6) (layer "F.Cu") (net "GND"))
 (segment (start 171.42 99.5) (end 175.02 103.1) (width 0.6) (layer "F.Cu") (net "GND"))
 (segment (start 162.35 83.616852) (end 164.770648 86.0375) (width 0.6) (layer "F.Cu") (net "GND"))
 (segment (start 165.0375 86) (end 165 86.0375) (width 0.6) (layer "F.Cu") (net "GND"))
 (segment (start 193.65 89.095) (end 194.5 88.245) (width 0.6) (layer "F.Cu") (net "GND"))
 (segment (start 166.5 68) (end 166 67.5) (width 0.6) (layer "F.Cu") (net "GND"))
 (segment (start 175.02 103.1) (end 194.955635 103.1) (width 0.6) (layer "F.Cu") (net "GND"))
 (segment (start 173 93.2625) (end 165.775 86.0375) (width 0.6) (layer "F.Cu") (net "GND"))
 (segment (start 194.65 84.85) (end 194.65 82.5) (width 0.6) (layer "F.Cu") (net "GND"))
 (segment (start 195.4 81.75) (end 195.4 73.608148) (width 0.6) (layer "F.Cu") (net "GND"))
 (segment (start 170.5 86) (end 165.0375 86) (width 0.6) (layer "F.Cu") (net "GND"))
 (segment (start 165.775 86.0375) (end 165 86.0375) (width 0.6) (layer "F.Cu") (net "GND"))
 (segment (start 194.791852 73) (end 166.5 73) (width 0.6) (layer "F.Cu") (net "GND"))
 (segment (start 162.35 77.5) (end 162.35 83.616852) (width 0.6) (layer "F.Cu") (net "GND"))
 (segment (start 171.42 99.5) (end 173 97.92) (width 0.6) (layer "F.Cu") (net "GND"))
 (segment (start 194.5 88.245) (end 194.5 85) (width 0.6) (layer "F.Cu") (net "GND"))
 (segment (start 194.955635 103.1) (end 198.6 99.455634) (width 0.6) (layer "F.Cu") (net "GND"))
 (segment (start 159.5 81.75) (end 159.5 68) (width 0.6) (layer "F.Cu") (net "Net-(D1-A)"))
 (segment (start 159.5 68) (end 159 67.5) (width 0.6) (layer "F.Cu") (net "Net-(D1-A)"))
 (segment (start 159.5 85.25) (end 161.15 83.6) (width 0.6) (layer "F.Cu") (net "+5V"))
 (segment (start 174 85.5) (end 172 83.5) (width 0.6) (layer "F.Cu") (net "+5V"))
 (segment (start 160.2875 91.7125) (end 159.5 90.925) (width 0.6) (layer "F.Cu") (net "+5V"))
 (segment (start 161.1 75.9) (end 161.5 75.5) (width 0.6) (layer "F.Cu") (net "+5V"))
 (segment (start 171.5 80) (end 167.5375 83.9625) (width 0.6) (layer "F.Cu") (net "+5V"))
 (segment (start 159.5 90.925) (end 159.5 85.25) (width 0.6) (layer "F.Cu") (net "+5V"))
 (segment (start 172 83.5) (end 172 80) (width 0.6) (layer "F.Cu") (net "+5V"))
 (segment (start 188 92.705) (end 188 87.97) (width 0.6) (layer "F.Cu") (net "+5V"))
 (segment (start 167.5375 83.9625) (end 165 83.9625) (width 0.6) (layer "F.Cu") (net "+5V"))
 (segment (start 164 75.5) (end 164 82.9625) (width 0.6) (layer "F.Cu") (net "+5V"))
 (segment (start 161.15 83.6) (end 161.15 79.15) (width 0.6) (layer "F.Cu") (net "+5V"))
 (segment (start 186.35 92.905) (end 187.8 92.905) (width 0.6) (layer "F.Cu") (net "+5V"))
 (segment (start 161.15 79.15) (end 161.1 79.1) (width 0.6) (layer "F.Cu") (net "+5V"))
 (segment (start 168.88 99.5) (end 162.275 92.895) (width 0.6) (layer "F.Cu") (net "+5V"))
 (segment (start 161.1 79.1) (end 161.1 75.9) (width 0.6) (layer "F.Cu") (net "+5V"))
 (segment (start 162.275 91.7125) (end 160.2875 91.7125) (width 0.6) (layer "F.Cu") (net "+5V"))
 (segment (start 188 87.97) (end 185.53 85.5) (width 0.6) (layer "F.Cu") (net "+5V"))
 (segment (start 162.275 92.895) (end 162.275 91.7125) (width 0.6) (layer "F.Cu") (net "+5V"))
 (segment (start 185.53 85.5) (end 174 85.5) (width 0.6) (layer "F.Cu") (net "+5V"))
 (segment (start 187.8 92.905) (end 188 92.705) (width 0.6) (layer "F.Cu") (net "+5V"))
 (segment (start 168.88 99.5) (end 169 99.5) (width 0.6) (layer "F.Cu") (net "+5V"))
 (segment (start 161.5 75.5) (end 164 75.5) (width 0.6) (layer "F.Cu") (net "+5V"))
 (segment (start 172 80) (end 171.5 80) (width 0.6) (layer "F.Cu") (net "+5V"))
 (segment (start 164 82.9625) (end 165 83.9625) (width 0.6) (layer "F.Cu") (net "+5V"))
 (segment (start 166.15 78) (end 165.65 77.5) (width 0.6) (layer "F.Cu") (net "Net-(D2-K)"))
 (segment (start 163.405635 73.35) (end 161.5 73.35) (width 0.6) (layer "F.Cu") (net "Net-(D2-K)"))
 (segment (start 172.5 77.5) (end 172 78) (width 0.6) (layer "F.Cu") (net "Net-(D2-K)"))
 (segment (start 179 77.5) (end 172.5 77.5) (width 0.6) (layer "F.Cu") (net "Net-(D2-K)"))
 (segment (start 161.5 73.35) (end 161.5 68) (width 0.6) (layer "F.Cu") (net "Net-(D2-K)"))
 (segment (start 172 78) (end 166.15 78) (width 0.6) (layer "F.Cu") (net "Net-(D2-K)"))
 (segment (start 165.65 77.5) (end 165.65 75.594365) (width 0.6) (layer "F.Cu") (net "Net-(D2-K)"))
 (segment (start 165.65 75.594365) (end 163.405635 73.35) (width 0.6) (layer "F.Cu") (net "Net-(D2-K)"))
 (segment (start 192 74.5) (end 166.15 74.5) (width 0.6) (layer "F.Cu") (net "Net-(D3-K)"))
 (segment (start 163.5 71.85) (end 163.5 68) (width 0.6) (layer "F.Cu") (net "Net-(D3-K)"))
 (segment (start 191.35 75.15) (end 192 74.5) (width 0.6) (layer "F.Cu") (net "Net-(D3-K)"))
 (segment (start 191.35 82.5) (end 191.35 75.15) (width 0.6) (layer "F.Cu") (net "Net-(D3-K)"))
 (segment (start 166.15 74.5) (end 163.5 71.85) (width 0.6) (layer "F.Cu") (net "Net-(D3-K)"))
 (segment (start 179.04 95.884366) (end 179.04 99.5) (width 0.6) (layer "F.Cu") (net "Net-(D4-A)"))
 (segment (start 177.3475 90.365) (end 186.35 90.365) (width 0.6) (layer "F.Cu") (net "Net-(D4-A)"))
 (segment (start 176.425 91.2875) (end 177.3475 90.365) (width 0.6) (layer "F.Cu") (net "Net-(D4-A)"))
 (segment (start 184.559366 90.365) (end 179.04 95.884366) (width 0.6) (layer "F.Cu") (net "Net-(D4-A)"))
 (segment (start 186.35 90.365) (end 184.559366 90.365) (width 0.6) (layer "F.Cu") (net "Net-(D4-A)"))
 (segment (start 173.625 91.2875) (end 173.625 91.125) (width 0.6) (layer "F.Cu") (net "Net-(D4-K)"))
 (segment (start 173.625 91.125) (end 170.5 88) (width 0.6) (layer "F.Cu") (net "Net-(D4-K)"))
 (segment (start 167.7125 91.7125) (end 171 95) (width 0.6) (layer "F.Cu") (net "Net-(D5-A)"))
 (segment (start 165.075 91.7125) (end 167.7125 91.7125) (width 0.6) (layer "F.Cu") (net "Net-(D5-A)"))
 (segment (start 175.5 89) (end 175.125 89.375) (width 0.6) (layer "F.Cu") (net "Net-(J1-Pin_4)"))
 (segment (start 186.35 89.095) (end 186.255 89) (width 0.6) (layer "F.Cu") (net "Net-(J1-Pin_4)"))
 (segment (start 175.125 89.375) (end 175.125 93.833148) (width 0.6) (layer "F.Cu") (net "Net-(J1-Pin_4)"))
 (segment (start 176.5 95.208148) (end 176.5 99.5) (width 0.6) (layer "F.Cu") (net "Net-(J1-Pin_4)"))
 (segment (start 175.125 93.833148) (end 176.5 95.208148) (width 0.6) (layer "F.Cu") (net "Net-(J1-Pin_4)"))
 (segment (start 186.255 89) (end 175.5 89) (width 0.6) (layer "F.Cu") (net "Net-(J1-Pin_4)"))
 (segment (start 190.635 91.635) (end 193.65 91.635) (width 0.6) (layer "F.Cu") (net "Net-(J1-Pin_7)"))
 (segment (start 190.5 87.5) (end 190.5 91.5) (width 0.6) (layer "F.Cu") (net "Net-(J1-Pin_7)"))
 (segment (start 190.5 91.5) (end 190.635 91.635) (width 0.6) (layer "F.Cu") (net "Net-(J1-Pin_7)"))
 (segment (start 179 79.5) (end 182.5 79.5) (width 0.6) (layer "F.Cu") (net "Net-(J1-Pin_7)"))
 (segment (start 179.5 79.5) (end 179 79.5) (width 0.6) (layer "F.Cu") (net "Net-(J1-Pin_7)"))
 (segment (start 182.5 79.5) (end 190.5 87.5) (width 0.6) (layer "F.Cu") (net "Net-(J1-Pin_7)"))
 (segment (start 191.985 91.635) (end 193.65 91.635) (width 0.6) (layer "F.Cu") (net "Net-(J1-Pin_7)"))
 (segment (start 184.12 99.5) (end 191.985 91.635) (width 0.6) (layer "F.Cu") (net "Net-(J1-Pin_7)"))
 (segment (start 183.5 92.98) (end 184.845 91.635) (width 0.6) (layer "F.Cu") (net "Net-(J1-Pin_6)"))
 (segment (start 183.5 97.58) (end 183.5 92.98) (width 0.6) (layer "F.Cu") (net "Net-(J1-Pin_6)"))
 (segment (start 181.58 99.5) (end 183.5 97.58) (width 0.6) (layer "F.Cu") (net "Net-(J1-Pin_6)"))
 (segment (start 184.845 91.635) (end 186.35 91.635) (width 0.6) (layer "F.Cu") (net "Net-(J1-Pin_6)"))
 (segment (start 189.2 99.5) (end 193.65 95.05) (width 0.6) (layer "F.Cu") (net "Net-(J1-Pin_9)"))
 (segment (start 193.65 95.05) (end 193.65 92.905) (width 0.6) (layer "F.Cu") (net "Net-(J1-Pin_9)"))
 (segment (start 194 75.2) (end 193 76.2) (width 0.6) (layer "F.Cu") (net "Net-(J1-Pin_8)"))
 (segment (start 194.5 102) (end 197.5 99) (width 0.6) (layer "F.Cu") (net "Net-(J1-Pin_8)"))
 (segment (start 189.16 102) (end 194.5 102) (width 0.6) (layer "F.Cu") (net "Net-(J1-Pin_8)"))
 (segment (start 195.865 90.365) (end 193.65 90.365) (width 0.6) (layer "F.Cu") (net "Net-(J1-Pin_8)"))
 (segment (start 193 86.97) (end 192 87.97) (width 0.6) (layer "F.Cu") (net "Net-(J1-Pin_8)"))
 (segment (start 192.145 90.365) (end 193.65 90.365) (width 0.6) (layer "F.Cu") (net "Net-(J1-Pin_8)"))
 (segment (start 186.66 99.5) (end 189.16 102) (width 0.6) (layer "F.Cu") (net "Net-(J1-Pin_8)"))
 (segment (start 197.5 92) (end 195.865 90.365) (width 0.6) (layer "F.Cu") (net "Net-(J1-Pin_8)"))
 (segment (start 194 74.5) (end 194 75.2) (width 0.6) (layer "F.Cu") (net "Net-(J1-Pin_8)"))
 (segment (start 197.5 99) (end 197.5 92) (width 0.6) (layer "F.Cu") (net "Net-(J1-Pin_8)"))
 (segment (start 192 90.22) (end 192.145 90.365) (width 0.6) (layer "F.Cu") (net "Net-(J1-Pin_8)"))
 (segment (start 192 87.97) (end 192 90.22) (width 0.6) (layer "F.Cu") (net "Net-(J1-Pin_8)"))
 (segment (start 193 76.2) (end 193 86.97) (width 0.6) (layer "F.Cu") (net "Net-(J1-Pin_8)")))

